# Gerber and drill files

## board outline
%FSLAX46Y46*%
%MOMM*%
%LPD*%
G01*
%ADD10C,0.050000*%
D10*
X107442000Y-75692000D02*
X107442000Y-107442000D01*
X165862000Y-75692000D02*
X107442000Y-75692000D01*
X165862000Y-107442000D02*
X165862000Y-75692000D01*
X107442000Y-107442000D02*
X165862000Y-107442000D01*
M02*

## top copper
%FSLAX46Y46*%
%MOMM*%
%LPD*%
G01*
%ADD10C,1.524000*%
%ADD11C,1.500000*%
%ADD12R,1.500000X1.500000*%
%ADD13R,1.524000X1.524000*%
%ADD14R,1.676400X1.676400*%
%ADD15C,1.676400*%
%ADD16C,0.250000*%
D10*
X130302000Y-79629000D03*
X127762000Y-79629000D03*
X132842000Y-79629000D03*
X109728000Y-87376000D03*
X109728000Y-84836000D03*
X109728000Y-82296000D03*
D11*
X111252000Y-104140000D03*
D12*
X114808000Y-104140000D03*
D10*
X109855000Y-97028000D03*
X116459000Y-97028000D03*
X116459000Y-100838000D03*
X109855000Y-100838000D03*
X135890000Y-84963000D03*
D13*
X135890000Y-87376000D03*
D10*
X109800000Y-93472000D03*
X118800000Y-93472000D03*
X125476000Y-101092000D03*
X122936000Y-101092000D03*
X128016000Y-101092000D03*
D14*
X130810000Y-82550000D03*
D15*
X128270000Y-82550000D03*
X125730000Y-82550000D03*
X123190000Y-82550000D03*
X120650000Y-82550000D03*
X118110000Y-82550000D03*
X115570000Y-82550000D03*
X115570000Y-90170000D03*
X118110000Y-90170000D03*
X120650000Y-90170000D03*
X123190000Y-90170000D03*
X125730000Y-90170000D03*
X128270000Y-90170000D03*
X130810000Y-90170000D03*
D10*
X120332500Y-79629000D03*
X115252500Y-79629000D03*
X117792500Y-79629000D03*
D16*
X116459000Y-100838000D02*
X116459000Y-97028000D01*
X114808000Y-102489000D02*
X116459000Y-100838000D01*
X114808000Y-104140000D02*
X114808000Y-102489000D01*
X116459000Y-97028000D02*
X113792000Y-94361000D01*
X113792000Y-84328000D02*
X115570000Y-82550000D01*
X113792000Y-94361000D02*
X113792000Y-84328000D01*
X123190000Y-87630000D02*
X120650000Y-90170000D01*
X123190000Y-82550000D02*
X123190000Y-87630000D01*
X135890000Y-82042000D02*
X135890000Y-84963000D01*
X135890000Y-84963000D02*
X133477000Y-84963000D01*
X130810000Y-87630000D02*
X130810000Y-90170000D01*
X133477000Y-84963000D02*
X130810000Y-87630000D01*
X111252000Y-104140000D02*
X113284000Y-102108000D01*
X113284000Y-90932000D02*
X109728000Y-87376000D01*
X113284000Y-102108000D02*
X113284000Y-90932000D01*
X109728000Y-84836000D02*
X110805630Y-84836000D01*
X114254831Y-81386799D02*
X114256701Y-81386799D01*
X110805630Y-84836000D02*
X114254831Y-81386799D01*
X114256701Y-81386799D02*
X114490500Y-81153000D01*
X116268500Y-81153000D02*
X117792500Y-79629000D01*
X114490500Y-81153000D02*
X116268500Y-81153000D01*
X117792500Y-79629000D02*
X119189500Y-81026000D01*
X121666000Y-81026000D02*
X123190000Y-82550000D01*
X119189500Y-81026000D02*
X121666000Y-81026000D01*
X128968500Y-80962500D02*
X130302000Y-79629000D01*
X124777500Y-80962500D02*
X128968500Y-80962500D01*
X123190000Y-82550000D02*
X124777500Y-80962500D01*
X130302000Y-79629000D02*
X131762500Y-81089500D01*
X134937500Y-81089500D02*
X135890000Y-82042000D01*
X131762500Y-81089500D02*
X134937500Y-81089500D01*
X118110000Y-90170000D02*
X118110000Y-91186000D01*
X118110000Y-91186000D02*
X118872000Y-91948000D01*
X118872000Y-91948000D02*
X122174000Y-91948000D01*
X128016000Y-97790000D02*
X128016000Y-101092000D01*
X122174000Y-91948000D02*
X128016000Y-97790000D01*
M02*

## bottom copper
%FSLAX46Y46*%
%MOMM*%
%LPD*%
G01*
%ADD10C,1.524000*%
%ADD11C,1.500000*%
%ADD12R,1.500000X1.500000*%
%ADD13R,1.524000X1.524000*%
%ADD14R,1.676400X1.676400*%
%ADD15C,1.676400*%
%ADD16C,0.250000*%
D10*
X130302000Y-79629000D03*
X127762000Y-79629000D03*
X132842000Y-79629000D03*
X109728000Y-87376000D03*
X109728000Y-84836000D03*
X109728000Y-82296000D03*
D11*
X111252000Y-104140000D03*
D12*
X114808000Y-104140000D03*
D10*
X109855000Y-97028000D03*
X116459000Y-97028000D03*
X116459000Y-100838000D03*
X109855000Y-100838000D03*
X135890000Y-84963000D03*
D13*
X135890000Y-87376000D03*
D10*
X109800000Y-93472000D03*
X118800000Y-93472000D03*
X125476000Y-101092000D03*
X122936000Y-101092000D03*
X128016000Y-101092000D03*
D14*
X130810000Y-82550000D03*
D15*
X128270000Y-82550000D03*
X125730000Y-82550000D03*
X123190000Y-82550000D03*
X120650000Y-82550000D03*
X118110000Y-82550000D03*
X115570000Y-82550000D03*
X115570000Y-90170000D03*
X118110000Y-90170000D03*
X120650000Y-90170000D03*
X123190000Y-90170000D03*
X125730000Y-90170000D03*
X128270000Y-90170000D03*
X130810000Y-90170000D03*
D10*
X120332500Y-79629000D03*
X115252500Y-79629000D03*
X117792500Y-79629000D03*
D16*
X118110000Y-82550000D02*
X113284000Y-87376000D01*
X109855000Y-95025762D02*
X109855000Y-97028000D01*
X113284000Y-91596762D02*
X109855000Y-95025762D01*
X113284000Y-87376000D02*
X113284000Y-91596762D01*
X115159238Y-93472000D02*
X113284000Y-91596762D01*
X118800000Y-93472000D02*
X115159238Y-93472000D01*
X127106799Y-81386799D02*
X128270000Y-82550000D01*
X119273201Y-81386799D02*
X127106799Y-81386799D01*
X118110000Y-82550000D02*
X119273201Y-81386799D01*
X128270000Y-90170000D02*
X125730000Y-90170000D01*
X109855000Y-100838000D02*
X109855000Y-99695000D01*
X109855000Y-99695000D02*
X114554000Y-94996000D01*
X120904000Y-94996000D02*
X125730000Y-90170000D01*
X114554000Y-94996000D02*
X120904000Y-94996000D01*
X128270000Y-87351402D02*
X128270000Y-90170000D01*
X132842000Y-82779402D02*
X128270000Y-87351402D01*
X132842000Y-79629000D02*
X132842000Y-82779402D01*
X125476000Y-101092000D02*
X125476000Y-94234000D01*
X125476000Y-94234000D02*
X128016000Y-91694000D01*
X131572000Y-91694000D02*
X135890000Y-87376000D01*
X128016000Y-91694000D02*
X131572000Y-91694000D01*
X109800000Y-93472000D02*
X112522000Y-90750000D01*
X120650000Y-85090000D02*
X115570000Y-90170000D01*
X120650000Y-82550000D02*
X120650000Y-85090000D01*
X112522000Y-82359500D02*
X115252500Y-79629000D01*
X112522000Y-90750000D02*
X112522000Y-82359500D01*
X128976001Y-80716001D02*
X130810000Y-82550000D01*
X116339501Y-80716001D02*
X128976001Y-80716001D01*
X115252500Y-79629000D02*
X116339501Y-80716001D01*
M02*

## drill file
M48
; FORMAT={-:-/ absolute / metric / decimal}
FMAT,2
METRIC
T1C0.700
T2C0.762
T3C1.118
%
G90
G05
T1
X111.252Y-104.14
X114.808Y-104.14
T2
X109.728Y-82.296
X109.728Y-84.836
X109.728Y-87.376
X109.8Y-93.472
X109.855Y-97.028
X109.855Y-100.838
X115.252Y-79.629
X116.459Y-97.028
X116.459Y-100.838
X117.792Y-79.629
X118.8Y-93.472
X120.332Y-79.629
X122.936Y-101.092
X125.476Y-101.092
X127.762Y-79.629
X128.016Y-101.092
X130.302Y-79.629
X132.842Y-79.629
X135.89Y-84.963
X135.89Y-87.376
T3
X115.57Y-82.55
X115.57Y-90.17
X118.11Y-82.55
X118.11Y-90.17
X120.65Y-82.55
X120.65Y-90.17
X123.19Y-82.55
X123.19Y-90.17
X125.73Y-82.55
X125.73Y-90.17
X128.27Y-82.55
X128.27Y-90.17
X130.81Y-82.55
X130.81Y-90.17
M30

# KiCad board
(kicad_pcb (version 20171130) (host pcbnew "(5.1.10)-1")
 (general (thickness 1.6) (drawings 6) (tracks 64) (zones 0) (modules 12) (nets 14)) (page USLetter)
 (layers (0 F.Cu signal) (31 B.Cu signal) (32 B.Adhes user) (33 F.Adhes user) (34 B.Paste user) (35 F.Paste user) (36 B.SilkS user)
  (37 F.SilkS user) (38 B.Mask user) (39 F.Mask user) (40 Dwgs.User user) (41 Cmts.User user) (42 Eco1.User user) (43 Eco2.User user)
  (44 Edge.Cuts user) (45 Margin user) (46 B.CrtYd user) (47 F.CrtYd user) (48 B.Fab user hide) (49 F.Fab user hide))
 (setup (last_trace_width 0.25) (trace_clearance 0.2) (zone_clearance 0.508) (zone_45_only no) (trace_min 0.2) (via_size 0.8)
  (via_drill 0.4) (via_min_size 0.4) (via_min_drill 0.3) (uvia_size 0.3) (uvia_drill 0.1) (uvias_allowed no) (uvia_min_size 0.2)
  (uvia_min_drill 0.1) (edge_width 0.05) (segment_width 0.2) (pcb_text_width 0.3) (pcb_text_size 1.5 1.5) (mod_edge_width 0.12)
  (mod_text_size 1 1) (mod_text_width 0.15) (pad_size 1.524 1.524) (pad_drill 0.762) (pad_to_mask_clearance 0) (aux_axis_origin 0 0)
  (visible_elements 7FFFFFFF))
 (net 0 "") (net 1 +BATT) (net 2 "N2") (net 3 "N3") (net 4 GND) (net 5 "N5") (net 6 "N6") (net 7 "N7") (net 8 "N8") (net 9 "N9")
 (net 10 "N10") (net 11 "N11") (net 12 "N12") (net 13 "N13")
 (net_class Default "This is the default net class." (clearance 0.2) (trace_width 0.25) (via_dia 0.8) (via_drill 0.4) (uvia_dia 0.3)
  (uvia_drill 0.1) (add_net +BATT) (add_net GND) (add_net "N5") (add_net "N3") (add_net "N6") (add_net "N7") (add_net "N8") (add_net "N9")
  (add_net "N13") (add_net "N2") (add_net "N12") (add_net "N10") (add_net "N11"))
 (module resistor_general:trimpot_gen (layer F.Cu) (at 130.302 80.645)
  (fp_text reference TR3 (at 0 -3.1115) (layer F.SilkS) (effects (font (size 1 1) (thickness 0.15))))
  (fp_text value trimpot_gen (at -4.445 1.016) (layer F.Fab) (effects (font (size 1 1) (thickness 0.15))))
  (pad 2 thru_hole circle (at 0 -1.016) (size 1.524 1.524) (drill 0.762) (layers *.Cu *.Mask) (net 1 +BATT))
  (pad 1 thru_hole circle (at -2.54 -1.016) (size 1.524 1.524) (drill 0.762) (layers *.Cu *.Mask) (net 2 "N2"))
  (pad 3 thru_hole circle (at 2.54 -1.016) (size 1.524 1.524) (drill 0.762) (layers *.Cu *.Mask) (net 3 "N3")))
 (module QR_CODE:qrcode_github (layer F.Cu) (at 154.178 86.614)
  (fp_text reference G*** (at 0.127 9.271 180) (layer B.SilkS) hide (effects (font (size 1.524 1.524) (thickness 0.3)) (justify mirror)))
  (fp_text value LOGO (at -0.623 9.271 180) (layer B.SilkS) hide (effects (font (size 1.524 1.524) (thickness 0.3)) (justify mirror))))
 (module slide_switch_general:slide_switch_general (layer F.Cu) (at 109.728 84.836 270)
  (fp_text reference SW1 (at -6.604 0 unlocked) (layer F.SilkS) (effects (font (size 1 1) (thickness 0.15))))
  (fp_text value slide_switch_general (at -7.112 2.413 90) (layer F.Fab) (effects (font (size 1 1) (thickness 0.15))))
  (pad 3 thru_hole circle (at 2.54 0 270) (size 1.524 1.524) (drill 0.762) (layers *.Cu *.Mask) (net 1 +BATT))
  (pad 2 thru_hole circle (at 0 0 270) (size 1.524 1.524) (drill 0.762) (layers *.Cu *.Mask) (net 1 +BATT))
  (pad 1 thru_hole circle (at -2.54 0 270) (size 1.524 1.524) (drill 0.762) (layers *.Cu *.Mask)))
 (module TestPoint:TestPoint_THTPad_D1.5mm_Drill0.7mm (layer F.Cu) (at 111.252 104.14)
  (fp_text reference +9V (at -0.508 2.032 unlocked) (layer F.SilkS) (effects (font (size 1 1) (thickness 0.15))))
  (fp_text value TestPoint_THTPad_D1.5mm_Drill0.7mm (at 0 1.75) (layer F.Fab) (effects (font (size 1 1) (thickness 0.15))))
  (pad 1 thru_hole circle (at 0 0) (size 1.5 1.5) (drill 0.7) (layers *.Cu *.Mask) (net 1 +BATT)))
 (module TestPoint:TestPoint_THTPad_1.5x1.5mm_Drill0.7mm (layer F.Cu) (at 114.808 104.14)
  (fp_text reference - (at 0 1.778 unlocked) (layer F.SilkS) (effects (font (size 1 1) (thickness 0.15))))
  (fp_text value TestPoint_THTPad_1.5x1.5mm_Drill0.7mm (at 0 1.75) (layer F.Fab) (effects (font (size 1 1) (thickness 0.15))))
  (pad 1 thru_hole rect (at 0 0) (size 1.5 1.5) (drill 0.7) (layers *.Cu *.Mask) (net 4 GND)))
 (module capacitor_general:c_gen (layer F.Cu) (at 113.284 97.028)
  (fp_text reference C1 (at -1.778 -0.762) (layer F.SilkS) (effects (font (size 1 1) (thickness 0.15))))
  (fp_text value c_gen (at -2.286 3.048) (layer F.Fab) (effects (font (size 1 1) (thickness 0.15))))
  (pad 1 thru_hole circle (at -3.429 0) (size 1.524 1.524) (drill 0.762) (layers *.Cu *.Mask) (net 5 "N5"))
  (pad 2 thru_hole circle (at 3.175 0) (size 1.524 1.524) (drill 0.762) (layers *.Cu *.Mask) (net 4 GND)))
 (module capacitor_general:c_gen (layer F.Cu) (at 113.284 100.838)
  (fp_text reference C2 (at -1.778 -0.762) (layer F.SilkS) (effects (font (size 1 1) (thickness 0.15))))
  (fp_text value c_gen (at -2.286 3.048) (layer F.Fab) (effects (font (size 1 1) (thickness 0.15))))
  (pad 2 thru_hole circle (at 3.175 0) (size 1.524 1.524) (drill 0.762) (layers *.Cu *.Mask) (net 4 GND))
  (pad 1 thru_hole circle (at -3.429 0) (size 1.524 1.524) (drill 0.762) (layers *.Cu *.Mask) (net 3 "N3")))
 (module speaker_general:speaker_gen (layer F.Cu) (at 135.89 86.106 270)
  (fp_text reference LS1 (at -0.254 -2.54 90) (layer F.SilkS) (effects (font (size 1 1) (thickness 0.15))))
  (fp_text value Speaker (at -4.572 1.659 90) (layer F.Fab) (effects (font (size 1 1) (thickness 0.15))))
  (pad 1 thru_hole circle (at -1.143 0 270) (size 1.524 1.524) (drill 0.762) (layers *.Cu *.Mask) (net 1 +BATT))
  (pad 2 thru_hole rect (at 1.27 0 270) (size 1.524 1.524) (drill 0.762) (layers *.Cu *.Mask) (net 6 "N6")))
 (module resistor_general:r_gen (layer F.Cu) (at 114.3 93.472)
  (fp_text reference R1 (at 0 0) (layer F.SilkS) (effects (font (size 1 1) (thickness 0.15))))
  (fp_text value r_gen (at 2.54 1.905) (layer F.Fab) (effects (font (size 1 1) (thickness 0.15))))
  (pad 1 thru_hole circle (at -4.5 0) (size 1.524 1.524) (drill 0.762) (layers *.Cu *.Mask) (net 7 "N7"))
  (pad 2 thru_hole circle (at 4.5 0) (size 1.524 1.524) (drill 0.762) (layers *.Cu *.Mask) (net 5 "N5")))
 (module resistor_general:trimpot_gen (layer F.Cu) (at 125.476 102.108)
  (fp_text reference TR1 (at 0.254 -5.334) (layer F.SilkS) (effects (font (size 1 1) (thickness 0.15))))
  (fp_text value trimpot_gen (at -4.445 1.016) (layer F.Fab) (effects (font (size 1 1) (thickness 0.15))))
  (pad 2 thru_hole circle (at 0 -1.016) (size 1.524 1.524) (drill 0.762) (layers *.Cu *.Mask) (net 6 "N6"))
  (pad 1 thru_hole circle (at -2.54 -1.016) (size 1.524 1.524) (drill 0.762) (layers *.Cu *.Mask) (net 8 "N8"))
  (pad 3 thru_hole circle (at 2.54 -1.016) (size 1.524 1.524) (drill 0.762) (layers *.Cu *.Mask) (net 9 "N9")))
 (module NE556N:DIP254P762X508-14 (layer F.Cu) (at 115.57 90.17 270)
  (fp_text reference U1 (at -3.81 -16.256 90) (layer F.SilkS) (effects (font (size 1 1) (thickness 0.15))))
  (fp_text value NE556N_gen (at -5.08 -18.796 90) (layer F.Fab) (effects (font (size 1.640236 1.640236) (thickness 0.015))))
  (pad 1 thru_hole rect (at -7.62 -15.24 270) (size 1.6764 1.6764) (drill 1.1176) (layers *.Cu *.Mask) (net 7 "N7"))
  (pad 2 thru_hole circle (at -7.62 -12.7 270) (size 1.6764 1.6764) (drill 1.1176) (layers *.Cu *.Mask) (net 5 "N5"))
  (pad 3 thru_hole circle (at -7.62 -10.16 270) (size 1.6764 1.6764) (drill 1.1176) (layers *.Cu *.Mask) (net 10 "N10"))
  (pad 4 thru_hole circle (at -7.62 -7.62 270) (size 1.6764 1.6764) (drill 1.1176) (layers *.Cu *.Mask) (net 1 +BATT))
  (pad 5 thru_hole circle (at -7.62 -5.08 270) (size 1.6764 1.6764) (drill 1.1176) (layers *.Cu *.Mask) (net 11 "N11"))
  (pad 6 thru_hole circle (at -7.62 -2.54 270) (size 1.6764 1.6764) (drill 1.1176) (layers *.Cu *.Mask) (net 5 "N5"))
  (pad 7 thru_hole circle (at -7.62 0 270) (size 1.6764 1.6764) (drill 1.1176) (layers *.Cu *.Mask) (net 4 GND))
  (pad 8 thru_hole circle (at 0 0 270) (size 1.6764 1.6764) (drill 1.1176) (layers *.Cu *.Mask) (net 11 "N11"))
  (pad 9 thru_hole circle (at 0 -2.54 270) (size 1.6764 1.6764) (drill 1.1176) (layers *.Cu *.Mask) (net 9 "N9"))
  (pad 10 thru_hole circle (at 0 -5.08 270) (size 1.6764 1.6764) (drill 1.1176) (layers *.Cu *.Mask) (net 1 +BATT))
  (pad 11 thru_hole circle (at 0 -7.62 270) (size 1.6764 1.6764) (drill 1.1176) (layers *.Cu *.Mask) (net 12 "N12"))
  (pad 12 thru_hole circle (at 0 -10.16 270) (size 1.6764 1.6764) (drill 1.1176) (layers *.Cu *.Mask) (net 3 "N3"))
  (pad 13 thru_hole circle (at 0 -12.7 270) (size 1.6764 1.6764) (drill 1.1176) (layers *.Cu *.Mask) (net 3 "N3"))
  (pad 14 thru_hole circle (at 0 -15.24 270) (size 1.6764 1.6764) (drill 1.1176) (layers *.Cu *.Mask) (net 1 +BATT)))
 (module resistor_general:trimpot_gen (layer F.Cu) (at 117.7925 80.645)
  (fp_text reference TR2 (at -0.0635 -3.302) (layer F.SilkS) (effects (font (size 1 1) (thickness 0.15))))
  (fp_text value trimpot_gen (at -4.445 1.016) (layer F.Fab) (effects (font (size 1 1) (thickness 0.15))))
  (pad 3 thru_hole circle (at 2.54 -1.016) (size 1.524 1.524) (drill 0.762) (layers *.Cu *.Mask) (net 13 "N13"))
  (pad 1 thru_hole circle (at -2.54 -1.016) (size 1.524 1.524) (drill 0.762) (layers *.Cu *.Mask) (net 7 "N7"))
  (pad 2 thru_hole circle (at 0 -1.016) (size 1.524 1.524) (drill 0.762) (layers *.Cu *.Mask) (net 1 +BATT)))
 (gr_line (start 107.442 75.692) (end 107.442 107.442) (layer Edge.Cuts) (width 0.05))
 (gr_line (start 165.862 75.692) (end 107.442 75.692) (layer Edge.Cuts) (width 0.05))
 (gr_line (start 165.862 107.442) (end 165.862 75.692) (layer Edge.Cuts) (width 0.05))
 (gr_line (start 107.442 107.442) (end 165.862 107.442) (layer Edge.Cuts) (width 0.05))
 (segment (start 118.11 82.55) (end 113.284 87.376) (width 0.25) (layer B.Cu) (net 5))
 (segment (start 109.855 95.025762) (end 109.855 97.028) (width 0.25) (layer B.Cu) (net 5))
 (segment (start 113.284 91.596762) (end 109.855 95.025762) (width 0.25) (layer B.Cu) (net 5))
 (segment (start 113.284 87.376) (end 113.284 91.596762) (width 0.25) (layer B.Cu) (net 5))
 (segment (start 115.159238 93.472) (end 113.284 91.596762) (width 0.25) (layer B.Cu) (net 5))
 (segment (start 118.8 93.472) (end 115.159238 93.472) (width 0.25) (layer B.Cu) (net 5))
 (segment (start 127.106799 81.386799) (end 128.27 82.55) (width 0.25) (layer B.Cu) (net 5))
 (segment (start 119.273201 81.386799) (end 127.106799 81.386799) (width 0.25) (layer B.Cu) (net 5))
 (segment (start 118.11 82.55) (end 119.273201 81.386799) (width 0.25) (layer B.Cu) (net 5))
 (segment (start 116.459 100.838) (end 116.459 97.028) (width 0.25) (layer F.Cu) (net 4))
 (segment (start 114.808 102.489) (end 116.459 100.838) (width 0.25) (layer F.Cu) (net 4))
 (segment (start 114.808 104.14) (end 114.808 102.489) (width 0.25) (layer F.Cu) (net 4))
 (segment (start 116.459 97.028) (end 113.792 94.361) (width 0.25) (layer F.Cu) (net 4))
 (segment (start 113.792 84.328) (end 115.57 82.55) (width 0.25) (layer F.Cu) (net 4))
 (segment (start 113.792 94.361) (end 113.792 84.328) (width 0.25) (layer F.Cu) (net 4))
 (segment (start 128.27 90.17) (end 125.73 90.17) (width 0.25) (layer B.Cu) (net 3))
 (segment (start 109.855 100.838) (end 109.855 99.695) (width 0.25) (layer B.Cu) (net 3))
 (segment (start 109.855 99.695) (end 114.554 94.996) (width 0.25) (layer B.Cu) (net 3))
 (segment (start 120.904 94.996) (end 125.73 90.17) (width 0.25) (layer B.Cu) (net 3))
 (segment (start 114.554 94.996) (end 120.904 94.996) (width 0.25) (layer B.Cu) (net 3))
 (segment (start 128.27 87.351402) (end 128.27 90.17) (width 0.25) (layer B.Cu) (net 3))
 (segment (start 132.842 82.779402) (end 128.27 87.351402) (width 0.25) (layer B.Cu) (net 3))
 (segment (start 132.842 79.629) (end 132.842 82.779402) (width 0.25) (layer B.Cu) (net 3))
 (segment (start 123.19 87.63) (end 120.65 90.17) (width 0.25) (layer F.Cu) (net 1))
 (segment (start 123.19 82.55) (end 123.19 87.63) (width 0.25) (layer F.Cu) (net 1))
 (segment (start 135.89 82.042) (end 135.89 84.963) (width 0.25) (layer F.Cu) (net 1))
 (segment (start 135.89 84.963) (end 133.477 84.963) (width 0.25) (layer F.Cu) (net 1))
 (segment (start 130.81 87.63) (end 130.81 90.17) (width 0.25) (layer F.Cu) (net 1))
 (segment (start 133.477 84.963) (end 130.81 87.63) (width 0.25) (layer F.Cu) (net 1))
 (segment (start 111.252 104.14) (end 113.284 102.108) (width 0.25) (layer F.Cu) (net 1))
 (segment (start 113.284 90.932) (end 109.728 87.376) (width 0.25) (layer F.Cu) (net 1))
 (segment (start 113.284 102.108) (end 113.284 90.932) (width 0.25) (layer F.Cu) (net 1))
 (segment (start 109.728 84.836) (end 110.80563 84.836) (width 0.25) (layer F.Cu) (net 1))
 (segment (start 114.254831 81.386799) (end 114.256701 81.386799) (width 0.25) (layer F.Cu) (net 1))
 (segment (start 110.80563 84.836) (end 114.254831 81.386799) (width 0.25) (layer F.Cu) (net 1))
 (segment (start 114.256701 81.386799) (end 114.4905 81.153) (width 0.25) (layer F.Cu) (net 1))
 (segment (start 116.2685 81.153) (end 117.7925 79.629) (width 0.25) (layer F.Cu) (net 1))
 (segment (start 114.4905 81.153) (end 116.2685 81.153) (width 0.25) (layer F.Cu) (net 1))
 (segment (start 117.7925 79.629) (end 119.1895 81.026) (width 0.25) (layer F.Cu) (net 1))
 (segment (start 121.666 81.026) (end 123.19 82.55) (width 0.25) (layer F.Cu) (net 1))
 (segment (start 119.1895 81.026) (end 121.666 81.026) (width 0.25) (layer F.Cu) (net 1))
 (segment (start 128.9685 80.9625) (end 130.302 79.629) (width 0.25) (layer F.Cu) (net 1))
 (segment (start 124.7775 80.9625) (end 128.9685 80.9625) (width 0.25) (layer F.Cu) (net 1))
 (segment (start 123.19 82.55) (end 124.7775 80.9625) (width 0.25) (layer F.Cu) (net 1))
 (segment (start 130.302 79.629) (end 131.7625 81.0895) (width 0.25) (layer F.Cu) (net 1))
 (segment (start 134.9375 81.0895) (end 135.89 82.042) (width 0.25) (layer F.Cu) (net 1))
 (segment (start 131.7625 81.0895) (end 134.9375 81.0895) (width 0.25) (layer F.Cu) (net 1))
 (segment (start 125.476 101.092) (end 125.476 94.234) (width 0.25) (layer B.Cu) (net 6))
 (segment (start 125.476 94.234) (end 128.016 91.694) (width 0.25) (layer B.Cu) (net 6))
 (segment (start 131.572 91.694) (end 135.89 87.376) (width 0.25) (layer B.Cu) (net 6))
 (segment (start 128.016 91.694) (end 131.572 91.694) (width 0.25) (layer B.Cu) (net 6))
 (segment (start 109.8 93.472) (end 112.522 90.75) (width 0.25) (layer B.Cu) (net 7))
 (segment (start 118.11 90.17) (end 118.11 91.186) (width 0.25) (layer F.Cu) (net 9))
 (segment (start 118.11 91.186) (end 118.872 91.948) (width 0.25) (layer F.Cu) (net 9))
 (segment (start 118.872 91.948) (end 122.174 91.948) (width 0.25) (layer F.Cu) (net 9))
 (segment (start 128.016 97.79) (end 128.016 101.092) (width 0.25) (layer F.Cu) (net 9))
 (segment (start 122.174 91.948) (end 128.016 97.79) (width 0.25) (layer F.Cu) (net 9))
 (segment (start 120.65 85.09) (end 115.57 90.17) (width 0.25) (layer B.Cu) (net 11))
 (segment (start 120.65 82.55) (end 120.65 85.09) (width 0.25) (layer B.Cu) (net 11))
 (segment (start 112.522 82.3595) (end 115.2525 79.629) (width 0.25) (layer B.Cu) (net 7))
 (segment (start 112.522 90.75) (end 112.522 82.3595) (width 0.25) (layer B.Cu) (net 7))
 (segment (start 128.976001 80.716001) (end 130.81 82.55) (width 0.25) (layer B.Cu) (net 7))
 (segment (start 116.339501 80.716001) (end 128.976001 80.716001) (width 0.25) (layer B.Cu) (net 7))
 (segment (start 115.2525 79.629) (end 116.339501 80.716001) (width 0.25) (layer B.Cu) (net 7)))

